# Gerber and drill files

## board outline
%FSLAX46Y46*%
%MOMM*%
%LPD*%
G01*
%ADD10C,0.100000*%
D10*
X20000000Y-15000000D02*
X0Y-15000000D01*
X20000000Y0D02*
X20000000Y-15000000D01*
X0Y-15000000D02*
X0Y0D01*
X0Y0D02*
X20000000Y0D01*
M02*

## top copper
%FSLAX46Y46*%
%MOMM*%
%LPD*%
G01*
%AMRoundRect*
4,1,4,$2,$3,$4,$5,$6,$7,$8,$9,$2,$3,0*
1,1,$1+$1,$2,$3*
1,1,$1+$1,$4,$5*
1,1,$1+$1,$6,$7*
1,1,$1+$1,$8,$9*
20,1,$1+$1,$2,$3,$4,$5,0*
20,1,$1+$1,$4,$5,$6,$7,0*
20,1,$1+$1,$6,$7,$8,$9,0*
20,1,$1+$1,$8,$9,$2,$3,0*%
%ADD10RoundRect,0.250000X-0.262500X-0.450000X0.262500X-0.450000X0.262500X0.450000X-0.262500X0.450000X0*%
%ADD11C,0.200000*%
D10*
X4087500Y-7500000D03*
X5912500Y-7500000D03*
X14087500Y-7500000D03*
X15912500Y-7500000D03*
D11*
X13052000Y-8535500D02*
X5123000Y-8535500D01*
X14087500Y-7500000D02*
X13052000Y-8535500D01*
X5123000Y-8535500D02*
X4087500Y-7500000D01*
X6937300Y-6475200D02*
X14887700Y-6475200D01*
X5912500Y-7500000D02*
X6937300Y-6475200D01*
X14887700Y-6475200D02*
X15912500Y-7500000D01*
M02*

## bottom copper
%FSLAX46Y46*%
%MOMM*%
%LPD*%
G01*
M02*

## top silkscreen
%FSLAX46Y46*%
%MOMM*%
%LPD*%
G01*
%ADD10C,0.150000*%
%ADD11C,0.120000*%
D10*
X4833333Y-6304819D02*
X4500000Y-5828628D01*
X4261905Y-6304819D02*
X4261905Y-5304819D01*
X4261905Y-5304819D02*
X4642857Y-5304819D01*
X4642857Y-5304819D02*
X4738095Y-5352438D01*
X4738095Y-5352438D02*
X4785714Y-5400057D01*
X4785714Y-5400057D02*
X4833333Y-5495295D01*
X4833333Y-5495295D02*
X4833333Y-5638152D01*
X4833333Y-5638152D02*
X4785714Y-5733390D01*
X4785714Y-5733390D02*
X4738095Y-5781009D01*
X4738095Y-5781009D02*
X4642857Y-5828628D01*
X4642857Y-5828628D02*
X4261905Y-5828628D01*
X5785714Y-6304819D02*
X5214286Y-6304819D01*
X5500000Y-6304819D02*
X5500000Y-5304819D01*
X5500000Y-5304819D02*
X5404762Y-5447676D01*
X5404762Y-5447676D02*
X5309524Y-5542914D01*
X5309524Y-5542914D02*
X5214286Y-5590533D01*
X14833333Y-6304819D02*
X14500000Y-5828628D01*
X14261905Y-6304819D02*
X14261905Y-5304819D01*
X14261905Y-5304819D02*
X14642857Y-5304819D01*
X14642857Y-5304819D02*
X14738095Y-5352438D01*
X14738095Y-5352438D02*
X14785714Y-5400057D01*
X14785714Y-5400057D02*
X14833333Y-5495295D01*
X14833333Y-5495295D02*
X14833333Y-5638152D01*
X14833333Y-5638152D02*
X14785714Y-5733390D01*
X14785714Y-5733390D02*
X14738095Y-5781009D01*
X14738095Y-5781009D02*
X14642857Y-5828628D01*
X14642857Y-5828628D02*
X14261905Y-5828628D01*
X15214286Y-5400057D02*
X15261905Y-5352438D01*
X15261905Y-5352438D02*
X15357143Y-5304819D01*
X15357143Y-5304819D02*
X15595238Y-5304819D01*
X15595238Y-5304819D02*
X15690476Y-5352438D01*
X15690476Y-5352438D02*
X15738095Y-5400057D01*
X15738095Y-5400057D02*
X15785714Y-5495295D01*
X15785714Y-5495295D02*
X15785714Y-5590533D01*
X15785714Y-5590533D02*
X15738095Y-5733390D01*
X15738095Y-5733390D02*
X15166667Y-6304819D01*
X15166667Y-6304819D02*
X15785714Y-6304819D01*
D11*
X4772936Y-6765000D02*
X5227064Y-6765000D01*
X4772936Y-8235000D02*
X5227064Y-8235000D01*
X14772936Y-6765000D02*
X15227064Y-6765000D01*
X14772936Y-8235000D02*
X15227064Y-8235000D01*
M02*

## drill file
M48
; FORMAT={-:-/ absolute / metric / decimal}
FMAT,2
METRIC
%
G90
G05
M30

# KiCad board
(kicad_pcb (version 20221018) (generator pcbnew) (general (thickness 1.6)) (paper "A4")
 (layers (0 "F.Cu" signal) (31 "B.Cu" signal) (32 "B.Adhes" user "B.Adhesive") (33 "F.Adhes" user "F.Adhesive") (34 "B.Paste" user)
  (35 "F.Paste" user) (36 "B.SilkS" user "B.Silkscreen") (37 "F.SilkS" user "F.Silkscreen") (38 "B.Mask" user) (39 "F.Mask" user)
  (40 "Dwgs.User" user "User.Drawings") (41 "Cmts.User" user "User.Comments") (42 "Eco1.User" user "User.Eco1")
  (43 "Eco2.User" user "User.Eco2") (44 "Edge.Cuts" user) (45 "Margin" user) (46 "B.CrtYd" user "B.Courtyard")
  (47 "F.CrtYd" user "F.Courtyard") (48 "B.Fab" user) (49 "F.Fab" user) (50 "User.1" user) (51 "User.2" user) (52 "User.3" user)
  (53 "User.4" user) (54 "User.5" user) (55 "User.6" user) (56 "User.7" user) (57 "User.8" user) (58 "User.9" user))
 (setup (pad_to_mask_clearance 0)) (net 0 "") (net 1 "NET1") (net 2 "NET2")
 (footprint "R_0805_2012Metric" (layer "F.Cu") (at 5 7.5)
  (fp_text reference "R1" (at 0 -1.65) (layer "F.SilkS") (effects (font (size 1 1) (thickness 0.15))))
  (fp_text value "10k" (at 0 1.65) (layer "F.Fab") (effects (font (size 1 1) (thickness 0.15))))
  (fp_line (start -0.227064 -0.735) (end 0.227064 -0.735) (stroke (width 0.12) (type solid)) (layer "F.SilkS"))
  (fp_line (start -0.227064 0.735) (end 0.227064 0.735) (stroke (width 0.12) (type solid)) (layer "F.SilkS"))
  (pad "1" smd roundrect (at -0.9125 0) (size 1.025 1.4) (layers "F.Cu" "F.Paste" "F.Mask") (roundrect_rratio 0.243902) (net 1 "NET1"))
  (pad "2" smd roundrect (at 0.9125 0) (size 1.025 1.4) (layers "F.Cu" "F.Paste" "F.Mask") (roundrect_rratio 0.243902) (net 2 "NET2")))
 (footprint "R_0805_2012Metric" (layer "F.Cu") (at 15 7.5)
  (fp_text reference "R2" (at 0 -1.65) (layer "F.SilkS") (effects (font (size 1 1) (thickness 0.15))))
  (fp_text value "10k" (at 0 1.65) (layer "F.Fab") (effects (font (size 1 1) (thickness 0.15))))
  (fp_line (start -0.227064 -0.735) (end 0.227064 -0.735) (stroke (width 0.12) (type solid)) (layer "F.SilkS"))
  (fp_line (start -0.227064 0.735) (end 0.227064 0.735) (stroke (width 0.12) (type solid)) (layer "F.SilkS"))
  (pad "1" smd roundrect (at -0.9125 0) (size 1.025 1.4) (layers "F.Cu" "F.Paste" "F.Mask") (roundrect_rratio 0.243902) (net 1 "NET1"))
  (pad "2" smd roundrect (at 0.9125 0) (size 1.025 1.4) (layers "F.Cu" "F.Paste" "F.Mask") (roundrect_rratio 0.243902) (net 2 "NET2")))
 (gr_line (start 20 15) (end 0 15) (stroke (width 0.1) (type default)) (layer "Edge.Cuts"))
 (gr_line (start 20 0) (end 20 15) (stroke (width 0.1) (type default)) (layer "Edge.Cuts"))
 (gr_line (start 0 15) (end 0 0) (stroke (width 0.1) (type default)) (layer "Edge.Cuts"))
 (gr_line (start 0 0) (end 20 0) (stroke (width 0.1) (type default)) (layer "Edge.Cuts"))
 (segment (start 13.052 8.5355) (end 5.123 8.5355) (width 0.2) (layer "F.Cu") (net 1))
 (segment (start 14.0875 7.5) (end 13.052 8.5355) (width 0.2) (layer "F.Cu") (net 1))
 (segment (start 5.123 8.5355) (end 4.0875 7.5) (width 0.2) (layer "F.Cu") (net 1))
 (segment (start 6.9373 6.4752) (end 14.8877 6.4752) (width 0.2) (layer "F.Cu") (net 2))
 (segment (start 5.9125 7.5) (end 6.9373 6.4752) (width 0.2) (layer "F.Cu") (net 2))
 (segment (start 14.8877 6.4752) (end 15.9125 7.5) (width 0.2) (layer "F.Cu") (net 2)))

